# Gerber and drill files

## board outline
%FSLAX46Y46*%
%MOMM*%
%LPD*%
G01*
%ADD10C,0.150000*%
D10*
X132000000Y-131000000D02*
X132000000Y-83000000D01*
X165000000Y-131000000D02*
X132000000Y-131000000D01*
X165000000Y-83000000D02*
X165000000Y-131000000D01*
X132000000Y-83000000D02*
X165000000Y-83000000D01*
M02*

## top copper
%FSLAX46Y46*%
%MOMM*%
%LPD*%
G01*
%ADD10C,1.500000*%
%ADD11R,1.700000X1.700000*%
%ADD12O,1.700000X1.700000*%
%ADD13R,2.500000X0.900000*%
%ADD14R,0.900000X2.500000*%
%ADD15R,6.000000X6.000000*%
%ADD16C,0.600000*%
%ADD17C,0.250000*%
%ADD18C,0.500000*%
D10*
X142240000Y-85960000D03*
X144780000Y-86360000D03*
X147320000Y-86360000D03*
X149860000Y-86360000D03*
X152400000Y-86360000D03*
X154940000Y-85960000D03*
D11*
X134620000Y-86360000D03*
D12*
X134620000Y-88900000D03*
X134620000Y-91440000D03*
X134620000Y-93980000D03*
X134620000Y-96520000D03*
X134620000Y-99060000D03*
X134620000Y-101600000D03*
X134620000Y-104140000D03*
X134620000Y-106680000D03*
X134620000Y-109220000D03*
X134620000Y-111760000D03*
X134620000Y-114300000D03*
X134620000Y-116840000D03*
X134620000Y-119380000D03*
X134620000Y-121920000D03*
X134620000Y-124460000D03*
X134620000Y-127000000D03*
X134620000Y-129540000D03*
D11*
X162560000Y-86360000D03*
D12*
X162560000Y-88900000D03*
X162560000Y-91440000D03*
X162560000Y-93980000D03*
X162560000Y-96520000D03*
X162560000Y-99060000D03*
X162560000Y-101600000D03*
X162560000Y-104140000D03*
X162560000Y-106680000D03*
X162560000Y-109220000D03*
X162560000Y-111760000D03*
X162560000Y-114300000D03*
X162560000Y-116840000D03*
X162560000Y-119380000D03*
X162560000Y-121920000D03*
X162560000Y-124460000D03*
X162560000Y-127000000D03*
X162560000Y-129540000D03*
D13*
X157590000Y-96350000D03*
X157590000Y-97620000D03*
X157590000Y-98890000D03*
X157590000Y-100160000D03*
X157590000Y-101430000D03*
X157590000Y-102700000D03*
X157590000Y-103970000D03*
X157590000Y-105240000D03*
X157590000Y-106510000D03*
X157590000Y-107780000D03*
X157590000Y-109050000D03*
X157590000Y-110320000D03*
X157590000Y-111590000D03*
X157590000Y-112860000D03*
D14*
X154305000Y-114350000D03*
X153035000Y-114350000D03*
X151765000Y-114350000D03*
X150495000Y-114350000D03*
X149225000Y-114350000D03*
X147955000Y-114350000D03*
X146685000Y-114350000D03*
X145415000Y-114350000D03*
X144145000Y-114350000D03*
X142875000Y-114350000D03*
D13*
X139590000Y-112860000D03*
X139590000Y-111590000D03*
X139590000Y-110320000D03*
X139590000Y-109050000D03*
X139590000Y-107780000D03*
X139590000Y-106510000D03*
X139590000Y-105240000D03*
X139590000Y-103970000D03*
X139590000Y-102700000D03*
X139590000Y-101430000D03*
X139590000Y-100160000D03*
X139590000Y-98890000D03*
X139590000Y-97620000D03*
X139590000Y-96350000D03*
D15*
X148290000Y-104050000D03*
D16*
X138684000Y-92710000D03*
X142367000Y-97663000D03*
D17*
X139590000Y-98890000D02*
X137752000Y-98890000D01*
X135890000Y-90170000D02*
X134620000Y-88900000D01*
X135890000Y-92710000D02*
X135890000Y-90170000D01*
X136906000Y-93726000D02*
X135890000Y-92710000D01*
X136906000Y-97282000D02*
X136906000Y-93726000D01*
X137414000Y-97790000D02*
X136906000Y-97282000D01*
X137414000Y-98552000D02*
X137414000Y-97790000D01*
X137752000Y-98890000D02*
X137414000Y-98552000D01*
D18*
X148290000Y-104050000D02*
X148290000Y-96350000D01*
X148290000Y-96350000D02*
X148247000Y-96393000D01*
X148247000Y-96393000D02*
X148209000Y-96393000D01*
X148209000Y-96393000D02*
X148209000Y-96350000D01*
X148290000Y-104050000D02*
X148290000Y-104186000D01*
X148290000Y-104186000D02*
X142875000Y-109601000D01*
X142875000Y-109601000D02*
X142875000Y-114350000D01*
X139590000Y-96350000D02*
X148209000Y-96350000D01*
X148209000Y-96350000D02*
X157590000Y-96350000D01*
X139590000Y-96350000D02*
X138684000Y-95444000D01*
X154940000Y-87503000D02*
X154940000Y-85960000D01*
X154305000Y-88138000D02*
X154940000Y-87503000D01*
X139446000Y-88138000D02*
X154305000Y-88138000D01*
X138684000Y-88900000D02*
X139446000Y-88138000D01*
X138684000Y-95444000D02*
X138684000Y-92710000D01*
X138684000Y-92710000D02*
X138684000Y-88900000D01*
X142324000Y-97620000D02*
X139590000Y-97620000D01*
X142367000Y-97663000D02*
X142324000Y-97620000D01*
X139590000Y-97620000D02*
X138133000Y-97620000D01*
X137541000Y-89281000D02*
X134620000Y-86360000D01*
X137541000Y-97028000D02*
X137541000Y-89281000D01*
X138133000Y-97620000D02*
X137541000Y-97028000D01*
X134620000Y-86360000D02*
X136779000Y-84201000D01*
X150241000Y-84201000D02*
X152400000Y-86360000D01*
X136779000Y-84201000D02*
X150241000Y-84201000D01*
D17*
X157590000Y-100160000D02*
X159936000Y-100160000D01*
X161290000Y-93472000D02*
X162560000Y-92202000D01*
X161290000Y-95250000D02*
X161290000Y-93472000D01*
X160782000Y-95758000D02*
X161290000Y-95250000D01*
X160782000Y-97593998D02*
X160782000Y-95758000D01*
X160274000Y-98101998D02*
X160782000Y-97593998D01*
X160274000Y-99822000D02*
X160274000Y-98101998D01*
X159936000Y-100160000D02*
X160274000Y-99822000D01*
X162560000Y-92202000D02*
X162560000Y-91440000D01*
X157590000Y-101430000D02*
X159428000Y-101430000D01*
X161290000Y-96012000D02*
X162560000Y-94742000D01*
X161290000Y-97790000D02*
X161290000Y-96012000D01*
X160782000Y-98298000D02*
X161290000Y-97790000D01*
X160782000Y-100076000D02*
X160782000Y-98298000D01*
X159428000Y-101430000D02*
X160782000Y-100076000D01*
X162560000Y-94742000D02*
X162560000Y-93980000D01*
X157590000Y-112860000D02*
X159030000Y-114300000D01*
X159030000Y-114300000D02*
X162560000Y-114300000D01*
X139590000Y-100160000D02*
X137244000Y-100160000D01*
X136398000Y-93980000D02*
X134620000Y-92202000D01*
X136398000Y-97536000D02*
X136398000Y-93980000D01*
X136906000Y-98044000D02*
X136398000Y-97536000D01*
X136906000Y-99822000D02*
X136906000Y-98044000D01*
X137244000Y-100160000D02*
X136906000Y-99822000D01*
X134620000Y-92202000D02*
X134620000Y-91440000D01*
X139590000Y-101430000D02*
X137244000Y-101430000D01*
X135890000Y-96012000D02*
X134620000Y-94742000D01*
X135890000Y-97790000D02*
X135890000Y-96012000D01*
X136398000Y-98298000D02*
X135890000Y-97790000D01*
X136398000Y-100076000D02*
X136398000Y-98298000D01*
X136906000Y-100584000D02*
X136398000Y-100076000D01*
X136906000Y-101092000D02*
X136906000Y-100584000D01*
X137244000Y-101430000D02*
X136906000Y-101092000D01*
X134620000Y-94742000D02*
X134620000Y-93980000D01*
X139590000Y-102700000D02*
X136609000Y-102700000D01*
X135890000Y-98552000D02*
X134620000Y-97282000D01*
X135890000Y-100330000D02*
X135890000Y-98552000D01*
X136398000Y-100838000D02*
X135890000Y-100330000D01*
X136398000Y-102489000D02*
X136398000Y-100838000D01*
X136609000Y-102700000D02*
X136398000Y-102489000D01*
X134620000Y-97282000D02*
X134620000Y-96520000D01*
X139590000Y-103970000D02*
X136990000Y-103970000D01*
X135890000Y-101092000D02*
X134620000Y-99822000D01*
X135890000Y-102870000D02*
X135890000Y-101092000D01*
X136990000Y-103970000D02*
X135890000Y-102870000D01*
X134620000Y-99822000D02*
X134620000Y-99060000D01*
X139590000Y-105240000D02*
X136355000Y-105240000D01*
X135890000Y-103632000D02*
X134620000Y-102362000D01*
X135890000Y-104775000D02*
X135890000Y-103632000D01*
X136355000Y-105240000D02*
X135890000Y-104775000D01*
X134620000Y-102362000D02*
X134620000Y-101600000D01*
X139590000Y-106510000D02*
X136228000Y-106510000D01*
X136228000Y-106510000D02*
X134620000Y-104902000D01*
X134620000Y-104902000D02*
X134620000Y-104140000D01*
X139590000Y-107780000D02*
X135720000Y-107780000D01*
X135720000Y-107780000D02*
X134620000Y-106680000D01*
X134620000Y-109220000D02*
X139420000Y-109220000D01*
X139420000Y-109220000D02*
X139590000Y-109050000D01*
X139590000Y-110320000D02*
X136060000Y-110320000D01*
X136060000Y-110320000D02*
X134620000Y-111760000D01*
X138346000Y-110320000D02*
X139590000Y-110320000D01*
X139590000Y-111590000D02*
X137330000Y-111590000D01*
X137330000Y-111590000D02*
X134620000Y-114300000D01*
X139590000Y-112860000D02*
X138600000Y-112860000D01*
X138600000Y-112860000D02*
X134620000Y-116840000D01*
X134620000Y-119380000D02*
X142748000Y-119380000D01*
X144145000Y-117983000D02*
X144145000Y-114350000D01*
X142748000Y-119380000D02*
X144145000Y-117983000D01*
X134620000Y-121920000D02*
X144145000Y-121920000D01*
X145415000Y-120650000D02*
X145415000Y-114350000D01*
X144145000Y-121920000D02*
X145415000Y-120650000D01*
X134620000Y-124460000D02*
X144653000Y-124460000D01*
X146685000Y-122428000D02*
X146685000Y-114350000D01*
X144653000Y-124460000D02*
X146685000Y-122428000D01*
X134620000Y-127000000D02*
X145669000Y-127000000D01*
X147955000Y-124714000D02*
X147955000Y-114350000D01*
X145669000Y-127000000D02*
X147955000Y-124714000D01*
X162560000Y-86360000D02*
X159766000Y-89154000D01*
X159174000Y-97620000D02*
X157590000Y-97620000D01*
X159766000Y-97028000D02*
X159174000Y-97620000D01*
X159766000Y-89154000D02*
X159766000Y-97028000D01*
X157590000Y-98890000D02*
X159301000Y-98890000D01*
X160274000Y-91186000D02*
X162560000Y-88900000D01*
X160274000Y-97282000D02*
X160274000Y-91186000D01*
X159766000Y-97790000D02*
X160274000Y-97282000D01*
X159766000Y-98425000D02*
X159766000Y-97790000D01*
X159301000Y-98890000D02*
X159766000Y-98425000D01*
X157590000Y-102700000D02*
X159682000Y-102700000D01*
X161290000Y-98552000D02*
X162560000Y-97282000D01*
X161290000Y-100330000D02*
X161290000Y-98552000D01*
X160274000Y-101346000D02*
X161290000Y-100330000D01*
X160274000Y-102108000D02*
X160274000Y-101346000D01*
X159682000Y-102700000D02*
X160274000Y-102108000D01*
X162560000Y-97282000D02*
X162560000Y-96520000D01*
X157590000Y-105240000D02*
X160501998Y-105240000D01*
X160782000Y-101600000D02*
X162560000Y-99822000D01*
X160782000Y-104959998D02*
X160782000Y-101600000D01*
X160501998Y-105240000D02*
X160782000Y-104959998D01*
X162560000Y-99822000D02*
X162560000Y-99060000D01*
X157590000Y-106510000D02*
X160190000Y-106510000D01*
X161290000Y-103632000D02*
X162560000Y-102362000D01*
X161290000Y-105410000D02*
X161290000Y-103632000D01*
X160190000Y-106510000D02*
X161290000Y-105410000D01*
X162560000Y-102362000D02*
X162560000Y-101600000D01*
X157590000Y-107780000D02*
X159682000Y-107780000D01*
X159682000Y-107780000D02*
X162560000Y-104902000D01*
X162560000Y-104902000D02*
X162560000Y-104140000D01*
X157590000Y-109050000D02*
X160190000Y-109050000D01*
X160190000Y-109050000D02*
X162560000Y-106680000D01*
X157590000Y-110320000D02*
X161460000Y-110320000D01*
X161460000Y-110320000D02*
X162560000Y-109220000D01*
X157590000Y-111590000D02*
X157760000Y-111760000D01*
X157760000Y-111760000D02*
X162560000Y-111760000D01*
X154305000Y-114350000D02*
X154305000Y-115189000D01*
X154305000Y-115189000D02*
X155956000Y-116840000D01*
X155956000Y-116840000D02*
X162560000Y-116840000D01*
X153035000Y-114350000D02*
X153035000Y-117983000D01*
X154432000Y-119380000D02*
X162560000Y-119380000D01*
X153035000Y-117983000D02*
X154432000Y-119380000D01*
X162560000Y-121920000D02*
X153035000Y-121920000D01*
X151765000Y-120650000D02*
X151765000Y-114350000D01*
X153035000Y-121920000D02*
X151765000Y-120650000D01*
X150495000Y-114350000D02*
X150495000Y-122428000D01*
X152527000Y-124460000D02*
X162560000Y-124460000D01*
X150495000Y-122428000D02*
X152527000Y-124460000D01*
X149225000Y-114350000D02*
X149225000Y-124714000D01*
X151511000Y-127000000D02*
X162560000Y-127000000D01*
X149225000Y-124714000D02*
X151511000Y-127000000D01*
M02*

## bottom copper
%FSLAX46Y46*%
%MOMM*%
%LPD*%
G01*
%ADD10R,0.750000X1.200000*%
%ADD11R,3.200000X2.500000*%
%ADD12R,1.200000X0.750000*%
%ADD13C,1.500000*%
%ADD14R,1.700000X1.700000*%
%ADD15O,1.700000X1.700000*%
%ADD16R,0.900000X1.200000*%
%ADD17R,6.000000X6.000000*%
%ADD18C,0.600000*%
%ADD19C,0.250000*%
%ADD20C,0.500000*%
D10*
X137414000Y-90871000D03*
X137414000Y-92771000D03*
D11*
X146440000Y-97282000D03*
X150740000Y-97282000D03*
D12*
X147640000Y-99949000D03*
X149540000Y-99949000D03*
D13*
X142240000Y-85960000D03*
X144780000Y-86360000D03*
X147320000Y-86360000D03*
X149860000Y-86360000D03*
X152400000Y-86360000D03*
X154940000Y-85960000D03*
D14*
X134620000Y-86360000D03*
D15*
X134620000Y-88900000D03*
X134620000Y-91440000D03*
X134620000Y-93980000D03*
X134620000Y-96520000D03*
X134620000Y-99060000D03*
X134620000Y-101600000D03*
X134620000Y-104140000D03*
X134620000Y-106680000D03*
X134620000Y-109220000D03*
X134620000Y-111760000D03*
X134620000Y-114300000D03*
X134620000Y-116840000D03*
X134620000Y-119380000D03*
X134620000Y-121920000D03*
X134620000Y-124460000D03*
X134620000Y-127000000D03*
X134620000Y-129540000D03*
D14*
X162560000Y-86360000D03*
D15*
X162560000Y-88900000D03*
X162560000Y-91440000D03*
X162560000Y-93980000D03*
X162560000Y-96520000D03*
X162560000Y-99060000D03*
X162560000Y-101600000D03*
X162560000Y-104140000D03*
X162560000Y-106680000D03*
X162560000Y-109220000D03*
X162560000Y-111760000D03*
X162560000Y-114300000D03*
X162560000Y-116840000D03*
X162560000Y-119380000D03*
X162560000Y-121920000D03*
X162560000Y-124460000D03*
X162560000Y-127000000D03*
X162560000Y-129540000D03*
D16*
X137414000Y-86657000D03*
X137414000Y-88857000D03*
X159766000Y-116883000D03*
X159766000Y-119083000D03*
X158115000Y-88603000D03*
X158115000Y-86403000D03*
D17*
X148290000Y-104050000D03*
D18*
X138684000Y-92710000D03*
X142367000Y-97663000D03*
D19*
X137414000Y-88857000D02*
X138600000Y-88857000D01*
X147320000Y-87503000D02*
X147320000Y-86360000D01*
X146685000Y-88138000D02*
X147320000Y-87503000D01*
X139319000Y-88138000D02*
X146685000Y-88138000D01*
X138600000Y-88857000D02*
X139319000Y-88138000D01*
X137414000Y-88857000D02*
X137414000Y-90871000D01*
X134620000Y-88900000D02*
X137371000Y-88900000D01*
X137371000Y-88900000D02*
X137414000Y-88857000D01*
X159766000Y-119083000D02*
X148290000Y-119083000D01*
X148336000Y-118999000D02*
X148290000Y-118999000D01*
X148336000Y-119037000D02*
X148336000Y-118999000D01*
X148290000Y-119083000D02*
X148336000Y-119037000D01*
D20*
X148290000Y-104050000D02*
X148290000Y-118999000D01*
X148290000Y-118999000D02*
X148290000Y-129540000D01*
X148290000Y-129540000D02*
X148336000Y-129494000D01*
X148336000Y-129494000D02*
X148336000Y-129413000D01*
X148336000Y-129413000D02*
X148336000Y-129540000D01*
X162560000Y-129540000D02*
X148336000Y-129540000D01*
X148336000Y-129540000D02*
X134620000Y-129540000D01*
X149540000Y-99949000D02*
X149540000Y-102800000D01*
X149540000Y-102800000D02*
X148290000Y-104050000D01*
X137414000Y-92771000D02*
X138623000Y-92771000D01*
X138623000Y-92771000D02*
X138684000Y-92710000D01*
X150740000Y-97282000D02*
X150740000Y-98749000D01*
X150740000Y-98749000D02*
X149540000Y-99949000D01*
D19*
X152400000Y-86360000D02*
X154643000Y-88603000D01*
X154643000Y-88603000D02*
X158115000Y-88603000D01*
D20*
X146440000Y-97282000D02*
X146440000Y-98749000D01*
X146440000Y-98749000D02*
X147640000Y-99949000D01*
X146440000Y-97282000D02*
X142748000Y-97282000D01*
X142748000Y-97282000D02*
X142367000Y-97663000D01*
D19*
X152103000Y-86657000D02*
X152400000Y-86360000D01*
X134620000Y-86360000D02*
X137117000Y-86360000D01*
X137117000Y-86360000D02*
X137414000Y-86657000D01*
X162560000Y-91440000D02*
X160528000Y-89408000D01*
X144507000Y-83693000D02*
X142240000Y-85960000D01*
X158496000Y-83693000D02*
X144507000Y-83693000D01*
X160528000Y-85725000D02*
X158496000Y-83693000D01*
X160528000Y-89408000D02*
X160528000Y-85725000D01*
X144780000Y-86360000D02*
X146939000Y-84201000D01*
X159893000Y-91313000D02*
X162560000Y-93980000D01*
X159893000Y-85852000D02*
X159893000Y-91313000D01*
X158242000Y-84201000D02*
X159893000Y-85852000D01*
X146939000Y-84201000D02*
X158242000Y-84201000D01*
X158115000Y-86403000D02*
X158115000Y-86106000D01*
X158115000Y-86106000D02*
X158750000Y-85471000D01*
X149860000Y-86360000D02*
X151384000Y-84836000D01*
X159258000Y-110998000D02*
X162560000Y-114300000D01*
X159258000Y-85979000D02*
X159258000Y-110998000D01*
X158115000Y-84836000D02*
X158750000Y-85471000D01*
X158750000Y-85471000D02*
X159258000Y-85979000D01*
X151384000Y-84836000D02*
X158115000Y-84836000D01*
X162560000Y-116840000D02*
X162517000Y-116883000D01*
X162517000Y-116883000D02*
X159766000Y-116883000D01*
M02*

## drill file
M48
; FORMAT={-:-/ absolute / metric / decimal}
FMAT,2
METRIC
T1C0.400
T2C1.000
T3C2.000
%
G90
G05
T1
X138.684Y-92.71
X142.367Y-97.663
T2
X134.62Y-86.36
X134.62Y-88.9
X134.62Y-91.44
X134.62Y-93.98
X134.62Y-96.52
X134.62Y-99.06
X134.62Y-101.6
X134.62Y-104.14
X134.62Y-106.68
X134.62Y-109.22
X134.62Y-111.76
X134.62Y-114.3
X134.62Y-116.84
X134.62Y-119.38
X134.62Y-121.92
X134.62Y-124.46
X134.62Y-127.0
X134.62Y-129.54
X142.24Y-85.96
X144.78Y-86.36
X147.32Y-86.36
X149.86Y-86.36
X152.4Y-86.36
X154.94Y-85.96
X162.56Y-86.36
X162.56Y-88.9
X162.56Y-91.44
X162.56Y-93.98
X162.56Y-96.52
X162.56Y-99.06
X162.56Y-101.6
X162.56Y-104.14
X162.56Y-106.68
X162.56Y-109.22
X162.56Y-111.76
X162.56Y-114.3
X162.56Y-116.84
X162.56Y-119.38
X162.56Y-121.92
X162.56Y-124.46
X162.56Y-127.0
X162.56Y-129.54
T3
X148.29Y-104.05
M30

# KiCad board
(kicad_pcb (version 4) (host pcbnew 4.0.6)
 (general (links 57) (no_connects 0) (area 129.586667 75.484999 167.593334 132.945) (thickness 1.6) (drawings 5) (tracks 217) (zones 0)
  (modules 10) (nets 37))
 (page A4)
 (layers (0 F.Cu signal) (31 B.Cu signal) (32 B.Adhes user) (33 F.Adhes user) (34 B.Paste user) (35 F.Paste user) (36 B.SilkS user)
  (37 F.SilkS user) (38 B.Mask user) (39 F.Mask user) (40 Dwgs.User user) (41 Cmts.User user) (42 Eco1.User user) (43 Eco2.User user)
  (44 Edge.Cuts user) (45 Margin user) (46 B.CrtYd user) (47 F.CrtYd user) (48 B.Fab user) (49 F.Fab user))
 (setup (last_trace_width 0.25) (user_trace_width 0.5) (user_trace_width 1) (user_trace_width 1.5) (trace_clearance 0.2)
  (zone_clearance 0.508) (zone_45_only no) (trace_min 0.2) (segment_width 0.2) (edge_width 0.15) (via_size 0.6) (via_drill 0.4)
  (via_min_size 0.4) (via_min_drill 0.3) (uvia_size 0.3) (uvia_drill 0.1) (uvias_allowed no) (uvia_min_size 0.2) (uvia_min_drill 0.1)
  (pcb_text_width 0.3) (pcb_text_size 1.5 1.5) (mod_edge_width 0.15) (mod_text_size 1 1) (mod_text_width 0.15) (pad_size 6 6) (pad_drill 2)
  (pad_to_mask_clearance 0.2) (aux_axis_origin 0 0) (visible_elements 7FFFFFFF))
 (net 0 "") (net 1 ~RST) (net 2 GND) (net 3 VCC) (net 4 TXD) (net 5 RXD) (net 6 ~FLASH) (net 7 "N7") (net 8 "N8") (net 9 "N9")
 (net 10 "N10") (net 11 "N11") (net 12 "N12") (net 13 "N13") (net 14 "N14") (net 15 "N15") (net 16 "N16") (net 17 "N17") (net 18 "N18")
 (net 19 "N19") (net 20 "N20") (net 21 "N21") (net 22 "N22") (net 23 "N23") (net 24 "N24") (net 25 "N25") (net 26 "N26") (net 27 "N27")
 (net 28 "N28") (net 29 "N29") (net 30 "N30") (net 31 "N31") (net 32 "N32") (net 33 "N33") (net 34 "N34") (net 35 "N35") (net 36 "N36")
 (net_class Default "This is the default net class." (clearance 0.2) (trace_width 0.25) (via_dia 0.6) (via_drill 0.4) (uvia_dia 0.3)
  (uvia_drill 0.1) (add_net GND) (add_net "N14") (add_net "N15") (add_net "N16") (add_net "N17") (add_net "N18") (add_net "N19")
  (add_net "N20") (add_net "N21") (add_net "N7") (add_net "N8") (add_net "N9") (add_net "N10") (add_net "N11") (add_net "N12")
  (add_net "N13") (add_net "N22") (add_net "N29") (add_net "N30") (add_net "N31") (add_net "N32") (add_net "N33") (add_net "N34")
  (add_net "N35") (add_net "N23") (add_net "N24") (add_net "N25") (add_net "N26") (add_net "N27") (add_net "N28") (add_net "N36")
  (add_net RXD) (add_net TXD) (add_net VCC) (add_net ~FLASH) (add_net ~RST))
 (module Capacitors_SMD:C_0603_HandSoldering (layer B.Cu) (at 137.414 91.821 270)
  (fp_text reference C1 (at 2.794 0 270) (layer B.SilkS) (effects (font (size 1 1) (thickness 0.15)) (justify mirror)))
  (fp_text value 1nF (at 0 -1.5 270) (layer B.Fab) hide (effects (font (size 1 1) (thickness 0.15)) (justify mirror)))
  (pad 1 smd rect (at -0.95 0 270) (size 1.2 0.75) (layers B.Cu B.Paste B.Mask) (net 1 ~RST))
  (pad 2 smd rect (at 0.95 0 270) (size 1.2 0.75) (layers B.Cu B.Paste B.Mask) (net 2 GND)))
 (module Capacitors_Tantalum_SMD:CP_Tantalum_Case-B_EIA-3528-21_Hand (layer B.Cu) (at 148.59 97.282)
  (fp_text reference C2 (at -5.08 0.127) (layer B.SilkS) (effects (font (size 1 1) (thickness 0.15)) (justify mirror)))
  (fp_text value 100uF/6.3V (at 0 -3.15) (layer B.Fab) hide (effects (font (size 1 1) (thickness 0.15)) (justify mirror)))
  (pad 1 smd rect (at -2.15 0) (size 3.2 2.5) (layers B.Cu B.Paste B.Mask) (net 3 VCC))
  (pad 2 smd rect (at 2.15 0) (size 3.2 2.5) (layers B.Cu B.Paste B.Mask) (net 2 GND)))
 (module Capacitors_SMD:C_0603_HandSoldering (layer B.Cu) (at 148.59 99.949)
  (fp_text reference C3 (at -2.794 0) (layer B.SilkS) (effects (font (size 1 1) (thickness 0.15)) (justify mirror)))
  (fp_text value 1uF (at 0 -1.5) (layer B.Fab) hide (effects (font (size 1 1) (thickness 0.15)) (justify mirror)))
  (pad 1 smd rect (at -0.95 0) (size 1.2 0.75) (layers B.Cu B.Paste B.Mask) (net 3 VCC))
  (pad 2 smd rect (at 0.95 0) (size 1.2 0.75) (layers B.Cu B.Paste B.Mask) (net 2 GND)))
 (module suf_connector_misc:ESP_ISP (layer F.Cu) (at 142.24 86.36 90)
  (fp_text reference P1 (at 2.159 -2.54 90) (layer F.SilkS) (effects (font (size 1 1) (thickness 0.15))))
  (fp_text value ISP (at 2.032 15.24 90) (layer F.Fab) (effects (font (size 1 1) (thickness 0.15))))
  (pad 1 thru_hole circle (at 0.4 0 90) (size 1.5 1.5) (drill 1) (layers *.Cu *.Mask) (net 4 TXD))
  (pad 2 thru_hole circle (at 0 2.54 90) (size 1.5 1.5) (drill 1) (layers *.Cu *.Mask) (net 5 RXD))
  (pad 3 thru_hole circle (at 0 5.08 90) (size 1.5 1.5) (drill 1) (layers *.Cu *.Mask) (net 1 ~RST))
  (pad 4 thru_hole circle (at 0 7.62 90) (size 1.5 1.5) (drill 1) (layers *.Cu *.Mask) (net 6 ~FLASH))
  (pad 5 thru_hole circle (at 0 10.16 90) (size 1.5 1.5) (drill 1) (layers *.Cu *.Mask) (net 3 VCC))
  (pad 6 thru_hole circle (at 0.4 12.7 90) (size 1.5 1.5) (drill 1) (layers *.Cu *.Mask) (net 2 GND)))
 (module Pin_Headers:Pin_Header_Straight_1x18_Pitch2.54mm (layer F.Cu) (at 134.62 86.36)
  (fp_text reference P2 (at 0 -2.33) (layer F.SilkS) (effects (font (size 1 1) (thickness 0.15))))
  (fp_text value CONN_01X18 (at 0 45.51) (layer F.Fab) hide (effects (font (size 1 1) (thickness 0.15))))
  (pad 1 thru_hole rect (at 0 0) (size 1.7 1.7) (drill 1) (layers *.Cu *.Mask) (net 3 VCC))
  (pad 2 thru_hole oval (at 0 2.54) (size 1.7 1.7) (drill 1) (layers *.Cu *.Mask) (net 1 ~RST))
  (pad 3 thru_hole oval (at 0 5.08) (size 1.7 1.7) (drill 1) (layers *.Cu *.Mask) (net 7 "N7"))
  (pad 4 thru_hole oval (at 0 7.62) (size 1.7 1.7) (drill 1) (layers *.Cu *.Mask) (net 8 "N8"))
  (pad 5 thru_hole oval (at 0 10.16) (size 1.7 1.7) (drill 1) (layers *.Cu *.Mask) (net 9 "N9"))
  (pad 6 thru_hole oval (at 0 12.7) (size 1.7 1.7) (drill 1) (layers *.Cu *.Mask) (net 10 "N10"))
  (pad 7 thru_hole oval (at 0 15.24) (size 1.7 1.7) (drill 1) (layers *.Cu *.Mask) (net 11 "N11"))
  (pad 8 thru_hole oval (at 0 17.78) (size 1.7 1.7) (drill 1) (layers *.Cu *.Mask) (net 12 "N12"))
  (pad 9 thru_hole oval (at 0 20.32) (size 1.7 1.7) (drill 1) (layers *.Cu *.Mask) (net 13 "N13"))
  (pad 10 thru_hole oval (at 0 22.86) (size 1.7 1.7) (drill 1) (layers *.Cu *.Mask) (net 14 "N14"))
  (pad 11 thru_hole oval (at 0 25.4) (size 1.7 1.7) (drill 1) (layers *.Cu *.Mask) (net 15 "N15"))
  (pad 12 thru_hole oval (at 0 27.94) (size 1.7 1.7) (drill 1) (layers *.Cu *.Mask) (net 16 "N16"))
  (pad 13 thru_hole oval (at 0 30.48) (size 1.7 1.7) (drill 1) (layers *.Cu *.Mask) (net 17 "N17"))
  (pad 14 thru_hole oval (at 0 33.02) (size 1.7 1.7) (drill 1) (layers *.Cu *.Mask) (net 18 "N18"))
  (pad 15 thru_hole oval (at 0 35.56) (size 1.7 1.7) (drill 1) (layers *.Cu *.Mask) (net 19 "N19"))
  (pad 16 thru_hole oval (at 0 38.1) (size 1.7 1.7) (drill 1) (layers *.Cu *.Mask) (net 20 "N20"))
  (pad 17 thru_hole oval (at 0 40.64) (size 1.7 1.7) (drill 1) (layers *.Cu *.Mask) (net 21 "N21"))
  (pad 18 thru_hole oval (at 0 43.18) (size 1.7 1.7) (drill 1) (layers *.Cu *.Mask) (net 2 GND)))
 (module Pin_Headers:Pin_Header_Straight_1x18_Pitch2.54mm (layer F.Cu) (at 162.56 86.36)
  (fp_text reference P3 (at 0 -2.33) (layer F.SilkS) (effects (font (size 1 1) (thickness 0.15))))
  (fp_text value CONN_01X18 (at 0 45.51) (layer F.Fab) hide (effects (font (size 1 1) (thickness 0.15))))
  (pad 1 thru_hole rect (at 0 0) (size 1.7 1.7) (drill 1) (layers *.Cu *.Mask) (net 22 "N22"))
  (pad 2 thru_hole oval (at 0 2.54) (size 1.7 1.7) (drill 1) (layers *.Cu *.Mask) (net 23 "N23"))
  (pad 3 thru_hole oval (at 0 5.08) (size 1.7 1.7) (drill 1) (layers *.Cu *.Mask) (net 4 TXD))
  (pad 4 thru_hole oval (at 0 7.62) (size 1.7 1.7) (drill 1) (layers *.Cu *.Mask) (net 5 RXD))
  (pad 5 thru_hole oval (at 0 10.16) (size 1.7 1.7) (drill 1) (layers *.Cu *.Mask) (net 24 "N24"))
  (pad 6 thru_hole oval (at 0 12.7) (size 1.7 1.7) (drill 1) (layers *.Cu *.Mask) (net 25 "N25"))
  (pad 7 thru_hole oval (at 0 15.24) (size 1.7 1.7) (drill 1) (layers *.Cu *.Mask) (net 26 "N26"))
  (pad 8 thru_hole oval (at 0 17.78) (size 1.7 1.7) (drill 1) (layers *.Cu *.Mask) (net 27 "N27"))
  (pad 9 thru_hole oval (at 0 20.32) (size 1.7 1.7) (drill 1) (layers *.Cu *.Mask) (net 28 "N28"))
  (pad 10 thru_hole oval (at 0 22.86) (size 1.7 1.7) (drill 1) (layers *.Cu *.Mask) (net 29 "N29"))
  (pad 11 thru_hole oval (at 0 25.4) (size 1.7 1.7) (drill 1) (layers *.Cu *.Mask) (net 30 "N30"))
  (pad 12 thru_hole oval (at 0 27.94) (size 1.7 1.7) (drill 1) (layers *.Cu *.Mask) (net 6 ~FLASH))
  (pad 13 thru_hole oval (at 0 30.48) (size 1.7 1.7) (drill 1) (layers *.Cu *.Mask) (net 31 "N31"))
  (pad 14 thru_hole oval (at 0 33.02) (size 1.7 1.7) (drill 1) (layers *.Cu *.Mask) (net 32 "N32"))
  (pad 15 thru_hole oval (at 0 35.56) (size 1.7 1.7) (drill 1) (layers *.Cu *.Mask) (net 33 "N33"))
  (pad 16 thru_hole oval (at 0 38.1) (size 1.7 1.7) (drill 1) (layers *.Cu *.Mask) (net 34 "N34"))
  (pad 17 thru_hole oval (at 0 40.64) (size 1.7 1.7) (drill 1) (layers *.Cu *.Mask) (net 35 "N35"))
  (pad 18 thru_hole oval (at 0 43.18) (size 1.7 1.7) (drill 1) (layers *.Cu *.Mask) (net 2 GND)))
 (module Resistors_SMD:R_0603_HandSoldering (layer B.Cu) (at 137.414 87.757 270)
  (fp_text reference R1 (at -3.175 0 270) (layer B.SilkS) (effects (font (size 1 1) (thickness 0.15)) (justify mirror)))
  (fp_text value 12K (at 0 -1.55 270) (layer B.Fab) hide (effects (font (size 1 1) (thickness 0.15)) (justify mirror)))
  (pad 1 smd rect (at -1.1 0 270) (size 1.2 0.9) (layers B.Cu B.Paste B.Mask) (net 3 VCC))
  (pad 2 smd rect (at 1.1 0 270) (size 1.2 0.9) (layers B.Cu B.Paste B.Mask) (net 1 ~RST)))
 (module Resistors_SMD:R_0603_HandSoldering (layer B.Cu) (at 159.766 117.983 270)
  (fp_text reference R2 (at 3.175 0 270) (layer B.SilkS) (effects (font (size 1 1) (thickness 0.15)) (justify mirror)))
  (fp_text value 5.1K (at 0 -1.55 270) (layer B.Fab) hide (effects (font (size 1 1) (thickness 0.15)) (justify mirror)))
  (pad 1 smd rect (at -1.1 0 270) (size 1.2 0.9) (layers B.Cu B.Paste B.Mask) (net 31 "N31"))
  (pad 2 smd rect (at 1.1 0 270) (size 1.2 0.9) (layers B.Cu B.Paste B.Mask) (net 2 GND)))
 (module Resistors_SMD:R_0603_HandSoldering (layer B.Cu) (at 158.115 87.503 90)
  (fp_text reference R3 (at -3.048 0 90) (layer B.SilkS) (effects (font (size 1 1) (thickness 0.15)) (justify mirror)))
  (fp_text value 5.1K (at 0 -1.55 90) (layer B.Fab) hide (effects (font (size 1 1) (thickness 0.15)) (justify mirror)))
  (pad 1 smd rect (at -1.1 0 90) (size 1.2 0.9) (layers B.Cu B.Paste B.Mask) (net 3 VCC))
  (pad 2 smd rect (at 1.1 0 90) (size 1.2 0.9) (layers B.Cu B.Paste B.Mask) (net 6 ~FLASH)))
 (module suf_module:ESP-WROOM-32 (layer F.Cu) (at 148.59 101.6 180)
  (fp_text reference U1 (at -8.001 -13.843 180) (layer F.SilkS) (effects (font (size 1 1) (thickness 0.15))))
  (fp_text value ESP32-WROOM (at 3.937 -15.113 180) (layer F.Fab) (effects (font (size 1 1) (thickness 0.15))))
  (pad 38 smd rect (at -9 5.25 180) (size 2.5 0.9) (layers F.Cu F.Paste F.Mask) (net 2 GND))
  (pad 37 smd rect (at -9 3.98 180) (size 2.5 0.9) (layers F.Cu F.Paste F.Mask) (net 22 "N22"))
  (pad 36 smd rect (at -9 2.71 180) (size 2.5 0.9) (layers F.Cu F.Paste F.Mask) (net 23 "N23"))
  (pad 35 smd rect (at -9 1.44 180) (size 2.5 0.9) (layers F.Cu F.Paste F.Mask) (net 4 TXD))
  (pad 34 smd rect (at -9 0.17 180) (size 2.5 0.9) (layers F.Cu F.Paste F.Mask) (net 5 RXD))
  (pad 33 smd rect (at -9 -1.1 180) (size 2.5 0.9) (layers F.Cu F.Paste F.Mask) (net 24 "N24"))
  (pad 32 smd rect (at -9 -2.37 180) (size 2.5 0.9) (layers F.Cu F.Paste F.Mask) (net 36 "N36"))
  (pad 31 smd rect (at -9 -3.64 180) (size 2.5 0.9) (layers F.Cu F.Paste F.Mask) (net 25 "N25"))
  (pad 30 smd rect (at -9 -4.91 180) (size 2.5 0.9) (layers F.Cu F.Paste F.Mask) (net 26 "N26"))
  (pad 29 smd rect (at -9 -6.18 180) (size 2.5 0.9) (layers F.Cu F.Paste F.Mask) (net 27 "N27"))
  (pad 28 smd rect (at -9 -7.45 180) (size 2.5 0.9) (layers F.Cu F.Paste F.Mask) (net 28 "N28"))
  (pad 27 smd rect (at -9 -8.72 180) (size 2.5 0.9) (layers F.Cu F.Paste F.Mask) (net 29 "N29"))
  (pad 26 smd rect (at -9 -9.99 180) (size 2.5 0.9) (layers F.Cu F.Paste F.Mask) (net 30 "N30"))
  (pad 25 smd rect (at -9 -11.26 180) (size 2.5 0.9) (layers F.Cu F.Paste F.Mask) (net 6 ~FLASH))
  (pad 24 smd rect (at -5.715 -12.75 180) (size 0.9 2.5) (layers F.Cu F.Paste F.Mask) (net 31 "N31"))
  (pad 23 smd rect (at -4.445 -12.75 180) (size 0.9 2.5) (layers F.Cu F.Paste F.Mask) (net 32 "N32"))
  (pad 22 smd rect (at -3.175 -12.75 180) (size 0.9 2.5) (layers F.Cu F.Paste F.Mask) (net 33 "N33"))
  (pad 21 smd rect (at -1.905 -12.75 180) (size 0.9 2.5) (layers F.Cu F.Paste F.Mask) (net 34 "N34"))
  (pad 20 smd rect (at -0.635 -12.75 180) (size 0.9 2.5) (layers F.Cu F.Paste F.Mask) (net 35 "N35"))
  (pad 19 smd rect (at 0.635 -12.75 180) (size 0.9 2.5) (layers F.Cu F.Paste F.Mask) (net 21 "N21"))
  (pad 18 smd rect (at 1.905 -12.75 180) (size 0.9 2.5) (layers F.Cu F.Paste F.Mask) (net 20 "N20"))
  (pad 17 smd rect (at 3.175 -12.75 180) (size 0.9 2.5) (layers F.Cu F.Paste F.Mask) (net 19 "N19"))
  (pad 16 smd rect (at 4.445 -12.75 180) (size 0.9 2.5) (layers F.Cu F.Paste F.Mask) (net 18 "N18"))
  (pad 15 smd rect (at 5.715 -12.75 180) (size 0.9 2.5) (layers F.Cu F.Paste F.Mask) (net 2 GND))
  (pad 14 smd rect (at 9 -11.26 180) (size 2.5 0.9) (layers F.Cu F.Paste F.Mask) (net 17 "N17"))
  (pad 13 smd rect (at 9 -9.99 180) (size 2.5 0.9) (layers F.Cu F.Paste F.Mask) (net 16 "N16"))
  (pad 12 smd rect (at 9 -8.72 180) (size 2.5 0.9) (layers F.Cu F.Paste F.Mask) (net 15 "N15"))
  (pad 11 smd rect (at 9 -7.45 180) (size 2.5 0.9) (layers F.Cu F.Paste F.Mask) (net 14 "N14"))
  (pad 10 smd rect (at 9 -6.18 180) (size 2.5 0.9) (layers F.Cu F.Paste F.Mask) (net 13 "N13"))
  (pad 9 smd rect (at 9 -4.91 180) (size 2.5 0.9) (layers F.Cu F.Paste F.Mask) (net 12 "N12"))
  (pad 8 smd rect (at 9 -3.64 180) (size 2.5 0.9) (layers F.Cu F.Paste F.Mask) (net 11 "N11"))
  (pad 7 smd rect (at 9 -2.37 180) (size 2.5 0.9) (layers F.Cu F.Paste F.Mask) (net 10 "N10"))
  (pad 6 smd rect (at 9 -1.1 180) (size 2.5 0.9) (layers F.Cu F.Paste F.Mask) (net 9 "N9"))
  (pad 5 smd rect (at 9 0.17 180) (size 2.5 0.9) (layers F.Cu F.Paste F.Mask) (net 8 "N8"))
  (pad 4 smd rect (at 9 1.44 180) (size 2.5 0.9) (layers F.Cu F.Paste F.Mask) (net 7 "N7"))
  (pad 3 smd rect (at 9 2.71 180) (size 2.5 0.9) (layers F.Cu F.Paste F.Mask) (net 1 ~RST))
  (pad 2 smd rect (at 9 3.98 180) (size 2.5 0.9) (layers F.Cu F.Paste F.Mask) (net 3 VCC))
  (pad 1 smd rect (at 9 5.25 180) (size 2.5 0.9) (layers F.Cu F.Paste F.Mask) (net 2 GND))
  (pad 39 thru_hole rect (at 0.3 -2.45 180) (size 6 6) (drill 2) (layers *.Cu *.Mask F.SilkS) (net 2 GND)))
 (gr_line (start 132 131) (end 132 83) (angle 90) (layer Edge.Cuts) (width 0.15))
 (gr_line (start 165 131) (end 132 131) (angle 90) (layer Edge.Cuts) (width 0.15))
 (gr_line (start 165 83) (end 165 131) (angle 90) (layer Edge.Cuts) (width 0.15))
 (gr_line (start 132 83) (end 165 83) (angle 90) (layer Edge.Cuts) (width 0.15))
 (segment (start 139.59 98.89) (end 137.752 98.89) (width 0.25) (layer F.Cu) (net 1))
 (segment (start 135.89 90.17) (end 134.62 88.9) (width 0.25) (layer F.Cu) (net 1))
 (segment (start 135.89 92.71) (end 135.89 90.17) (width 0.25) (layer F.Cu) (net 1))
 (segment (start 136.906 93.726) (end 135.89 92.71) (width 0.25) (layer F.Cu) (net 1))
 (segment (start 136.906 97.282) (end 136.906 93.726) (width 0.25) (layer F.Cu) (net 1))
 (segment (start 137.414 97.79) (end 136.906 97.282) (width 0.25) (layer F.Cu) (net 1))
 (segment (start 137.414 98.552) (end 137.414 97.79) (width 0.25) (layer F.Cu) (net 1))
 (segment (start 137.752 98.89) (end 137.414 98.552) (width 0.25) (layer F.Cu) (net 1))
 (segment (start 137.414 88.857) (end 138.6 88.857) (width 0.25) (layer B.Cu) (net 1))
 (segment (start 147.32 87.503) (end 147.32 86.36) (width 0.25) (layer B.Cu) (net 1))
 (segment (start 146.685 88.138) (end 147.32 87.503) (width 0.25) (layer B.Cu) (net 1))
 (segment (start 139.319 88.138) (end 146.685 88.138) (width 0.25) (layer B.Cu) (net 1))
 (segment (start 138.6 88.857) (end 139.319 88.138) (width 0.25) (layer B.Cu) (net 1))
 (segment (start 137.414 88.857) (end 137.414 90.871) (width 0.25) (layer B.Cu) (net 1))
 (segment (start 134.62 88.9) (end 137.371 88.9) (width 0.25) (layer B.Cu) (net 1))
 (segment (start 137.371 88.9) (end 137.414 88.857) (width 0.25) (layer B.Cu) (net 1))
 (segment (start 148.29 104.05) (end 148.29 96.35) (width 0.5) (layer F.Cu) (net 2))
 (segment (start 148.29 96.35) (end 148.247 96.393) (width 0.5) (layer F.Cu) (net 2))
 (segment (start 148.247 96.393) (end 148.209 96.393) (width 0.5) (layer F.Cu) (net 2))
 (segment (start 148.209 96.393) (end 148.209 96.35) (width 0.5) (layer F.Cu) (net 2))
 (segment (start 159.766 119.083) (end 148.29 119.083) (width 0.25) (layer B.Cu) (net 2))
 (segment (start 148.336 118.999) (end 148.29 118.999) (width 0.25) (layer B.Cu) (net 2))
 (segment (start 148.336 119.037) (end 148.336 118.999) (width 0.25) (layer B.Cu) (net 2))
 (segment (start 148.29 119.083) (end 148.336 119.037) (width 0.25) (layer B.Cu) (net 2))
 (segment (start 148.29 104.05) (end 148.29 118.999) (width 0.5) (layer B.Cu) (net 2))
 (segment (start 148.29 118.999) (end 148.29 129.54) (width 0.5) (layer B.Cu) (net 2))
 (segment (start 148.29 129.54) (end 148.336 129.494) (width 0.5) (layer B.Cu) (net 2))
 (segment (start 148.336 129.494) (end 148.336 129.413) (width 0.5) (layer B.Cu) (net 2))
 (segment (start 148.336 129.413) (end 148.336 129.54) (width 0.5) (layer B.Cu) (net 2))
 (segment (start 162.56 129.54) (end 148.336 129.54) (width 0.5) (layer B.Cu) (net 2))
 (segment (start 148.336 129.54) (end 134.62 129.54) (width 0.5) (layer B.Cu) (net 2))
 (segment (start 148.29 104.05) (end 148.29 104.186) (width 0.5) (layer F.Cu) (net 2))
 (segment (start 148.29 104.186) (end 142.875 109.601) (width 0.5) (layer F.Cu) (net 2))
 (segment (start 142.875 109.601) (end 142.875 114.35) (width 0.5) (layer F.Cu) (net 2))
 (segment (start 149.54 99.949) (end 149.54 102.8) (width 0.5) (layer B.Cu) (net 2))
 (segment (start 149.54 102.8) (end 148.29 104.05) (width 0.5) (layer B.Cu) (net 2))
 (segment (start 137.414 92.771) (end 138.623 92.771) (width 0.5) (layer B.Cu) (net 2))
 (via (at 138.684 92.71) (size 0.6) (drill 0.4) (layers F.Cu B.Cu) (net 2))
 (segment (start 138.623 92.771) (end 138.684 92.71) (width 0.5) (layer B.Cu) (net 2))
 (segment (start 139.59 96.35) (end 148.209 96.35) (width 0.5) (layer F.Cu) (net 2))
 (segment (start 148.209 96.35) (end 157.59 96.35) (width 0.5) (layer F.Cu) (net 2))
 (segment (start 150.74 97.282) (end 150.74 98.749) (width 0.5) (layer B.Cu) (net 2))
 (segment (start 150.74 98.749) (end 149.54 99.949) (width 0.5) (layer B.Cu) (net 2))
 (segment (start 139.59 96.35) (end 138.684 95.444) (width 0.5) (layer F.Cu) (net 2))
 (segment (start 154.94 87.503) (end 154.94 85.96) (width 0.5) (layer F.Cu) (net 2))
 (segment (start 154.305 88.138) (end 154.94 87.503) (width 0.5) (layer F.Cu) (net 2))
 (segment (start 139.446 88.138) (end 154.305 88.138) (width 0.5) (layer F.Cu) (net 2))
 (segment (start 138.684 88.9) (end 139.446 88.138) (width 0.5) (layer F.Cu) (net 2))
 (segment (start 138.684 95.444) (end 138.684 92.71) (width 0.5) (layer F.Cu) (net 2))
 (segment (start 138.684 92.71) (end 138.684 88.9) (width 0.5) (layer F.Cu) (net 2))
 (segment (start 152.4 86.36) (end 154.643 88.603) (width 0.25) (layer B.Cu) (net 3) (status 400000))
 (segment (start 154.643 88.603) (end 158.115 88.603) (width 0.25) (layer B.Cu) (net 3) (status 800000))
 (segment (start 146.44 97.282) (end 146.44 98.749) (width 0.5) (layer B.Cu) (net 3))
 (segment (start 146.44 98.749) (end 147.64 99.949) (width 0.5) (layer B.Cu) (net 3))
 (segment (start 146.44 97.282) (end 142.748 97.282) (width 0.5) (layer B.Cu) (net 3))
 (segment (start 142.324 97.62) (end 139.59 97.62) (width 0.5) (layer F.Cu) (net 3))
 (segment (start 142.367 97.663) (end 142.324 97.62) (width 0.5) (layer F.Cu) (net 3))
 (via (at 142.367 97.663) (size 0.6) (drill 0.4) (layers F.Cu B.Cu) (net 3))
 (segment (start 142.748 97.282) (end 142.367 97.663) (width 0.5) (layer B.Cu) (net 3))
 (segment (start 139.59 97.62) (end 138.133 97.62) (width 0.5) (layer F.Cu) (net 3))
 (segment (start 137.541 89.281) (end 134.62 86.36) (width 0.5) (layer F.Cu) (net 3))
 (segment (start 137.541 97.028) (end 137.541 89.281) (width 0.5) (layer F.Cu) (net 3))
 (segment (start 138.133 97.62) (end 137.541 97.028) (width 0.5) (layer F.Cu) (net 3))
 (segment (start 152.103 86.657) (end 152.4 86.36) (width 0.25) (layer B.Cu) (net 3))
 (segment (start 134.62 86.36) (end 136.779 84.201) (width 0.5) (layer F.Cu) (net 3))
 (segment (start 150.241 84.201) (end 152.4 86.36) (width 0.5) (layer F.Cu) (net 3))
 (segment (start 136.779 84.201) (end 150.241 84.201) (width 0.5) (layer F.Cu) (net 3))
 (segment (start 134.62 86.36) (end 137.117 86.36) (width 0.25) (layer B.Cu) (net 3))
 (segment (start 137.117 86.36) (end 137.414 86.657) (width 0.25) (layer B.Cu) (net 3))
 (segment (start 162.56 91.44) (end 160.528 89.408) (width 0.25) (layer B.Cu) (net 4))
 (segment (start 144.507 83.693) (end 142.24 85.96) (width 0.25) (layer B.Cu) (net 4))
 (segment (start 158.496 83.693) (end 144.507 83.693) (width 0.25) (layer B.Cu) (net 4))
 (segment (start 160.528 85.725) (end 158.496 83.693) (width 0.25) (layer B.Cu) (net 4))
 (segment (start 160.528 89.408) (end 160.528 85.725) (width 0.25) (layer B.Cu) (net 4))
 (segment (start 157.59 100.16) (end 159.936 100.16) (width 0.25) (layer F.Cu) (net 4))
 (segment (start 161.29 93.472) (end 162.56 92.202) (width 0.25) (layer F.Cu) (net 4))
 (segment (start 161.29 95.25) (end 161.29 93.472) (width 0.25) (layer F.Cu) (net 4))
 (segment (start 160.782 95.758) (end 161.29 95.25) (width 0.25) (layer F.Cu) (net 4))
 (segment (start 160.782 97.593998) (end 160.782 95.758) (width 0.25) (layer F.Cu) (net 4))
 (segment (start 160.274 98.101998) (end 160.782 97.593998) (width 0.25) (layer F.Cu) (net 4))
 (segment (start 160.274 99.822) (end 160.274 98.101998) (width 0.25) (layer F.Cu) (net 4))
 (segment (start 159.936 100.16) (end 160.274 99.822) (width 0.25) (layer F.Cu) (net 4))
 (segment (start 162.56 92.202) (end 162.56 91.44) (width 0.25) (layer F.Cu) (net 4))
 (segment (start 144.78 86.36) (end 146.939 84.201) (width 0.25) (layer B.Cu) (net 5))
 (segment (start 159.893 91.313) (end 162.56 93.98) (width 0.25) (layer B.Cu) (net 5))
 (segment (start 159.893 85.852) (end 159.893 91.313) (width 0.25) (layer B.Cu) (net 5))
 (segment (start 158.242 84.201) (end 159.893 85.852) (width 0.25) (layer B.Cu) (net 5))
 (segment (start 146.939 84.201) (end 158.242 84.201) (width 0.25) (layer B.Cu) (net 5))
 (segment (start 157.59 101.43) (end 159.428 101.43) (width 0.25) (layer F.Cu) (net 5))
 (segment (start 161.29 96.012) (end 162.56 94.742) (width 0.25) (layer F.Cu) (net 5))
 (segment (start 161.29 97.79) (end 161.29 96.012) (width 0.25) (layer F.Cu) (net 5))
 (segment (start 160.782 98.298) (end 161.29 97.79) (width 0.25) (layer F.Cu) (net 5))
 (segment (start 160.782 100.076) (end 160.782 98.298) (width 0.25) (layer F.Cu) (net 5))
 (segment (start 159.428 101.43) (end 160.782 100.076) (width 0.25) (layer F.Cu) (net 5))
 (segment (start 162.56 94.742) (end 162.56 93.98) (width 0.25) (layer F.Cu) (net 5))
 (segment (start 158.115 86.403) (end 158.115 86.106) (width 0.25) (layer B.Cu) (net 6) (status C00000))
 (segment (start 158.115 86.106) (end 158.75 85.471) (width 0.25) (layer B.Cu) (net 6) (status 400000))
 (segment (start 149.86 86.36) (end 151.384 84.836) (width 0.25) (layer B.Cu) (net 6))
 (segment (start 159.258 110.998) (end 162.56 114.3) (width 0.25) (layer B.Cu) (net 6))
 (segment (start 159.258 85.979) (end 159.258 110.998) (width 0.25) (layer B.Cu) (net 6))
 (segment (start 158.115 84.836) (end 158.75 85.471) (width 0.25) (layer B.Cu) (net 6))
 (segment (start 158.75 85.471) (end 159.258 85.979) (width 0.25) (layer B.Cu) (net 6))
 (segment (start 151.384 84.836) (end 158.115 84.836) (width 0.25) (layer B.Cu) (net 6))
 (segment (start 157.59 112.86) (end 159.03 114.3) (width 0.25) (layer F.Cu) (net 6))
 (segment (start 159.03 114.3) (end 162.56 114.3) (width 0.25) (layer F.Cu) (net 6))
 (segment (start 139.59 100.16) (end 137.244 100.16) (width 0.25) (layer F.Cu) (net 7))
 (segment (start 136.398 93.98) (end 134.62 92.202) (width 0.25) (layer F.Cu) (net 7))
 (segment (start 136.398 97.536) (end 136.398 93.98) (width 0.25) (layer F.Cu) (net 7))
 (segment (start 136.906 98.044) (end 136.398 97.536) (width 0.25) (layer F.Cu) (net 7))
 (segment (start 136.906 99.822) (end 136.906 98.044) (width 0.25) (layer F.Cu) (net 7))
 (segment (start 137.244 100.16) (end 136.906 99.822) (width 0.25) (layer F.Cu) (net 7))
 (segment (start 134.62 92.202) (end 134.62 91.44) (width 0.25) (layer F.Cu) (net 7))
 (segment (start 139.59 101.43) (end 137.244 101.43) (width 0.25) (layer F.Cu) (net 8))
 (segment (start 135.89 96.012) (end 134.62 94.742) (width 0.25) (layer F.Cu) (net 8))
 (segment (start 135.89 97.79) (end 135.89 96.012) (width 0.25) (layer F.Cu) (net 8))
 (segment (start 136.398 98.298) (end 135.89 97.79) (width 0.25) (layer F.Cu) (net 8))
 (segment (start 136.398 100.076) (end 136.398 98.298) (width 0.25) (layer F.Cu) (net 8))
 (segment (start 136.906 100.584) (end 136.398 100.076) (width 0.25) (layer F.Cu) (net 8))
 (segment (start 136.906 101.092) (end 136.906 100.584) (width 0.25) (layer F.Cu) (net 8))
 (segment (start 137.244 101.43) (end 136.906 101.092) (width 0.25) (layer F.Cu) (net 8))
 (segment (start 134.62 94.742) (end 134.62 93.98) (width 0.25) (layer F.Cu) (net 8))
 (segment (start 139.59 102.7) (end 136.609 102.7) (width 0.25) (layer F.Cu) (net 9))
 (segment (start 135.89 98.552) (end 134.62 97.282) (width 0.25) (layer F.Cu) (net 9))
 (segment (start 135.89 100.33) (end 135.89 98.552) (width 0.25) (layer F.Cu) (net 9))
 (segment (start 136.398 100.838) (end 135.89 100.33) (width 0.25) (layer F.Cu) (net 9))
 (segment (start 136.398 102.489) (end 136.398 100.838) (width 0.25) (layer F.Cu) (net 9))
 (segment (start 136.609 102.7) (end 136.398 102.489) (width 0.25) (layer F.Cu) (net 9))
 (segment (start 134.62 97.282) (end 134.62 96.52) (width 0.25) (layer F.Cu) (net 9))
 (segment (start 139.59 103.97) (end 136.99 103.97) (width 0.25) (layer F.Cu) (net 10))
 (segment (start 135.89 101.092) (end 134.62 99.822) (width 0.25) (layer F.Cu) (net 10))
 (segment (start 135.89 102.87) (end 135.89 101.092) (width 0.25) (layer F.Cu) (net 10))
 (segment (start 136.99 103.97) (end 135.89 102.87) (width 0.25) (layer F.Cu) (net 10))
 (segment (start 134.62 99.822) (end 134.62 99.06) (width 0.25) (layer F.Cu) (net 10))
 (segment (start 139.59 105.24) (end 136.355 105.24) (width 0.25) (layer F.Cu) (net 11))
 (segment (start 135.89 103.632) (end 134.62 102.362) (width 0.25) (layer F.Cu) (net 11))
 (segment (start 135.89 104.775) (end 135.89 103.632) (width 0.25) (layer F.Cu) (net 11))
 (segment (start 136.355 105.24) (end 135.89 104.775) (width 0.25) (layer F.Cu) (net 11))
 (segment (start 134.62 102.362) (end 134.62 101.6) (width 0.25) (layer F.Cu) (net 11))
 (segment (start 139.59 106.51) (end 136.228 106.51) (width 0.25) (layer F.Cu) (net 12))
 (segment (start 136.228 106.51) (end 134.62 104.902) (width 0.25) (layer F.Cu) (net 12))
 (segment (start 134.62 104.902) (end 134.62 104.14) (width 0.25) (layer F.Cu) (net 12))
 (segment (start 139.59 107.78) (end 135.72 107.78) (width 0.25) (layer F.Cu) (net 13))
 (segment (start 135.72 107.78) (end 134.62 106.68) (width 0.25) (layer F.Cu) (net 13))
 (segment (start 134.62 109.22) (end 139.42 109.22) (width 0.25) (layer F.Cu) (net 14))
 (segment (start 139.42 109.22) (end 139.59 109.05) (width 0.25) (layer F.Cu) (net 14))
 (segment (start 139.59 110.32) (end 136.06 110.32) (width 0.25) (layer F.Cu) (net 15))
 (segment (start 136.06 110.32) (end 134.62 111.76) (width 0.25) (layer F.Cu) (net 15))
 (segment (start 138.346 110.32) (end 139.59 110.32) (width 0.25) (layer F.Cu) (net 15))
 (segment (start 139.59 111.59) (end 137.33 111.59) (width 0.25) (layer F.Cu) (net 16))
 (segment (start 137.33 111.59) (end 134.62 114.3) (width 0.25) (layer F.Cu) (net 16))
 (segment (start 139.59 112.86) (end 138.6 112.86) (width 0.25) (layer F.Cu) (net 17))
 (segment (start 138.6 112.86) (end 134.62 116.84) (width 0.25) (layer F.Cu) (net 17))
 (segment (start 134.62 119.38) (end 142.748 119.38) (width 0.25) (layer F.Cu) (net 18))
 (segment (start 144.145 117.983) (end 144.145 114.35) (width 0.25) (layer F.Cu) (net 18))
 (segment (start 142.748 119.38) (end 144.145 117.983) (width 0.25) (layer F.Cu) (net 18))
 (segment (start 134.62 121.92) (end 144.145 121.92) (width 0.25) (layer F.Cu) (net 19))
 (segment (start 145.415 120.65) (end 145.415 114.35) (width 0.25) (layer F.Cu) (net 19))
 (segment (start 144.145 121.92) (end 145.415 120.65) (width 0.25) (layer F.Cu) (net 19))
 (segment (start 134.62 124.46) (end 144.653 124.46) (width 0.25) (layer F.Cu) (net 20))
 (segment (start 146.685 122.428) (end 146.685 114.35) (width 0.25) (layer F.Cu) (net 20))
 (segment (start 144.653 124.46) (end 146.685 122.428) (width 0.25) (layer F.Cu) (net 20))
 (segment (start 134.62 127) (end 145.669 127) (width 0.25) (layer F.Cu) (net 21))
 (segment (start 147.955 124.714) (end 147.955 114.35) (width 0.25) (layer F.Cu) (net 21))
 (segment (start 145.669 127) (end 147.955 124.714) (width 0.25) (layer F.Cu) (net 21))
 (segment (start 162.56 86.36) (end 159.766 89.154) (width 0.25) (layer F.Cu) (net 22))
 (segment (start 159.174 97.62) (end 157.59 97.62) (width 0.25) (layer F.Cu) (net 22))
 (segment (start 159.766 97.028) (end 159.174 97.62) (width 0.25) (layer F.Cu) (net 22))
 (segment (start 159.766 89.154) (end 159.766 97.028) (width 0.25) (layer F.Cu) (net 22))
 (segment (start 157.59 98.89) (end 159.301 98.89) (width 0.25) (layer F.Cu) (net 23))
 (segment (start 160.274 91.186) (end 162.56 88.9) (width 0.25) (layer F.Cu) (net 23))
 (segment (start 160.274 97.282) (end 160.274 91.186) (width 0.25) (layer F.Cu) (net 23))
 (segment (start 159.766 97.79) (end 160.274 97.282) (width 0.25) (layer F.Cu) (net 23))
 (segment (start 159.766 98.425) (end 159.766 97.79) (width 0.25) (layer F.Cu) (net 23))
 (segment (start 159.301 98.89) (end 159.766 98.425) (width 0.25) (layer F.Cu) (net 23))
 (segment (start 157.59 102.7) (end 159.682 102.7) (width 0.25) (layer F.Cu) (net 24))
 (segment (start 161.29 98.552) (end 162.56 97.282) (width 0.25) (layer F.Cu) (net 24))
 (segment (start 161.29 100.33) (end 161.29 98.552) (width 0.25) (layer F.Cu) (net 24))
 (segment (start 160.274 101.346) (end 161.29 100.33) (width 0.25) (layer F.Cu) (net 24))
 (segment (start 160.274 102.108) (end 160.274 101.346) (width 0.25) (layer F.Cu) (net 24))
 (segment (start 159.682 102.7) (end 160.274 102.108) (width 0.25) (layer F.Cu) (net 24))
 (segment (start 162.56 97.282) (end 162.56 96.52) (width 0.25) (layer F.Cu) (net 24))
 (segment (start 157.59 105.24) (end 160.501998 105.24) (width 0.25) (layer F.Cu) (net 25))
 (segment (start 160.782 101.6) (end 162.56 99.822) (width 0.25) (layer F.Cu) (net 25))
 (segment (start 160.782 104.959998) (end 160.782 101.6) (width 0.25) (layer F.Cu) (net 25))
 (segment (start 160.501998 105.24) (end 160.782 104.959998) (width 0.25) (layer F.Cu) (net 25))
 (segment (start 162.56 99.822) (end 162.56 99.06) (width 0.25) (layer F.Cu) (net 25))
 (segment (start 157.59 106.51) (end 160.19 106.51) (width 0.25) (layer F.Cu) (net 26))
 (segment (start 161.29 103.632) (end 162.56 102.362) (width 0.25) (layer F.Cu) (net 26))
 (segment (start 161.29 105.41) (end 161.29 103.632) (width 0.25) (layer F.Cu) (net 26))
 (segment (start 160.19 106.51) (end 161.29 105.41) (width 0.25) (layer F.Cu) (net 26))
 (segment (start 162.56 102.362) (end 162.56 101.6) (width 0.25) (layer F.Cu) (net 26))
 (segment (start 157.59 107.78) (end 159.682 107.78) (width 0.25) (layer F.Cu) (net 27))
 (segment (start 159.682 107.78) (end 162.56 104.902) (width 0.25) (layer F.Cu) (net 27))
 (segment (start 162.56 104.902) (end 162.56 104.14) (width 0.25) (layer F.Cu) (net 27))
 (segment (start 157.59 109.05) (end 160.19 109.05) (width 0.25) (layer F.Cu) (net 28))
 (segment (start 160.19 109.05) (end 162.56 106.68) (width 0.25) (layer F.Cu) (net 28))
 (segment (start 157.59 110.32) (end 161.46 110.32) (width 0.25) (layer F.Cu) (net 29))
 (segment (start 161.46 110.32) (end 162.56 109.22) (width 0.25) (layer F.Cu) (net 29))
 (segment (start 157.59 111.59) (end 157.76 111.76) (width 0.25) (layer F.Cu) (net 30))
 (segment (start 157.76 111.76) (end 162.56 111.76) (width 0.25) (layer F.Cu) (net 30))
 (segment (start 162.56 116.84) (end 162.517 116.883) (width 0.25) (layer B.Cu) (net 31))
 (segment (start 162.517 116.883) (end 159.766 116.883) (width 0.25) (layer B.Cu) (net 31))
 (segment (start 154.305 114.35) (end 154.305 115.189) (width 0.25) (layer F.Cu) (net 31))
 (segment (start 154.305 115.189) (end 155.956 116.84) (width 0.25) (layer F.Cu) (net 31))
 (segment (start 155.956 116.84) (end 162.56 116.84) (width 0.25) (layer F.Cu) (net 31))
 (segment (start 153.035 114.35) (end 153.035 117.983) (width 0.25) (layer F.Cu) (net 32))
 (segment (start 154.432 119.38) (end 162.56 119.38) (width 0.25) (layer F.Cu) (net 32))
 (segment (start 153.035 117.983) (end 154.432 119.38) (width 0.25) (layer F.Cu) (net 32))
 (segment (start 162.56 121.92) (end 153.035 121.92) (width 0.25) (layer F.Cu) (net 33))
 (segment (start 151.765 120.65) (end 151.765 114.35) (width 0.25) (layer F.Cu) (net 33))
 (segment (start 153.035 121.92) (end 151.765 120.65) (width 0.25) (layer F.Cu) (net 33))
 (segment (start 150.495 114.35) (end 150.495 122.428) (width 0.25) (layer F.Cu) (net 34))
 (segment (start 152.527 124.46) (end 162.56 124.46) (width 0.25) (layer F.Cu) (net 34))
 (segment (start 150.495 122.428) (end 152.527 124.46) (width 0.25) (layer F.Cu) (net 34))
 (segment (start 149.225 114.35) (end 149.225 124.714) (width 0.25) (layer F.Cu) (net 35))
 (segment (start 151.511 127) (end 162.56 127) (width 0.25) (layer F.Cu) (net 35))
 (segment (start 149.225 124.714) (end 151.511 127) (width 0.25) (layer F.Cu) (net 35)))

